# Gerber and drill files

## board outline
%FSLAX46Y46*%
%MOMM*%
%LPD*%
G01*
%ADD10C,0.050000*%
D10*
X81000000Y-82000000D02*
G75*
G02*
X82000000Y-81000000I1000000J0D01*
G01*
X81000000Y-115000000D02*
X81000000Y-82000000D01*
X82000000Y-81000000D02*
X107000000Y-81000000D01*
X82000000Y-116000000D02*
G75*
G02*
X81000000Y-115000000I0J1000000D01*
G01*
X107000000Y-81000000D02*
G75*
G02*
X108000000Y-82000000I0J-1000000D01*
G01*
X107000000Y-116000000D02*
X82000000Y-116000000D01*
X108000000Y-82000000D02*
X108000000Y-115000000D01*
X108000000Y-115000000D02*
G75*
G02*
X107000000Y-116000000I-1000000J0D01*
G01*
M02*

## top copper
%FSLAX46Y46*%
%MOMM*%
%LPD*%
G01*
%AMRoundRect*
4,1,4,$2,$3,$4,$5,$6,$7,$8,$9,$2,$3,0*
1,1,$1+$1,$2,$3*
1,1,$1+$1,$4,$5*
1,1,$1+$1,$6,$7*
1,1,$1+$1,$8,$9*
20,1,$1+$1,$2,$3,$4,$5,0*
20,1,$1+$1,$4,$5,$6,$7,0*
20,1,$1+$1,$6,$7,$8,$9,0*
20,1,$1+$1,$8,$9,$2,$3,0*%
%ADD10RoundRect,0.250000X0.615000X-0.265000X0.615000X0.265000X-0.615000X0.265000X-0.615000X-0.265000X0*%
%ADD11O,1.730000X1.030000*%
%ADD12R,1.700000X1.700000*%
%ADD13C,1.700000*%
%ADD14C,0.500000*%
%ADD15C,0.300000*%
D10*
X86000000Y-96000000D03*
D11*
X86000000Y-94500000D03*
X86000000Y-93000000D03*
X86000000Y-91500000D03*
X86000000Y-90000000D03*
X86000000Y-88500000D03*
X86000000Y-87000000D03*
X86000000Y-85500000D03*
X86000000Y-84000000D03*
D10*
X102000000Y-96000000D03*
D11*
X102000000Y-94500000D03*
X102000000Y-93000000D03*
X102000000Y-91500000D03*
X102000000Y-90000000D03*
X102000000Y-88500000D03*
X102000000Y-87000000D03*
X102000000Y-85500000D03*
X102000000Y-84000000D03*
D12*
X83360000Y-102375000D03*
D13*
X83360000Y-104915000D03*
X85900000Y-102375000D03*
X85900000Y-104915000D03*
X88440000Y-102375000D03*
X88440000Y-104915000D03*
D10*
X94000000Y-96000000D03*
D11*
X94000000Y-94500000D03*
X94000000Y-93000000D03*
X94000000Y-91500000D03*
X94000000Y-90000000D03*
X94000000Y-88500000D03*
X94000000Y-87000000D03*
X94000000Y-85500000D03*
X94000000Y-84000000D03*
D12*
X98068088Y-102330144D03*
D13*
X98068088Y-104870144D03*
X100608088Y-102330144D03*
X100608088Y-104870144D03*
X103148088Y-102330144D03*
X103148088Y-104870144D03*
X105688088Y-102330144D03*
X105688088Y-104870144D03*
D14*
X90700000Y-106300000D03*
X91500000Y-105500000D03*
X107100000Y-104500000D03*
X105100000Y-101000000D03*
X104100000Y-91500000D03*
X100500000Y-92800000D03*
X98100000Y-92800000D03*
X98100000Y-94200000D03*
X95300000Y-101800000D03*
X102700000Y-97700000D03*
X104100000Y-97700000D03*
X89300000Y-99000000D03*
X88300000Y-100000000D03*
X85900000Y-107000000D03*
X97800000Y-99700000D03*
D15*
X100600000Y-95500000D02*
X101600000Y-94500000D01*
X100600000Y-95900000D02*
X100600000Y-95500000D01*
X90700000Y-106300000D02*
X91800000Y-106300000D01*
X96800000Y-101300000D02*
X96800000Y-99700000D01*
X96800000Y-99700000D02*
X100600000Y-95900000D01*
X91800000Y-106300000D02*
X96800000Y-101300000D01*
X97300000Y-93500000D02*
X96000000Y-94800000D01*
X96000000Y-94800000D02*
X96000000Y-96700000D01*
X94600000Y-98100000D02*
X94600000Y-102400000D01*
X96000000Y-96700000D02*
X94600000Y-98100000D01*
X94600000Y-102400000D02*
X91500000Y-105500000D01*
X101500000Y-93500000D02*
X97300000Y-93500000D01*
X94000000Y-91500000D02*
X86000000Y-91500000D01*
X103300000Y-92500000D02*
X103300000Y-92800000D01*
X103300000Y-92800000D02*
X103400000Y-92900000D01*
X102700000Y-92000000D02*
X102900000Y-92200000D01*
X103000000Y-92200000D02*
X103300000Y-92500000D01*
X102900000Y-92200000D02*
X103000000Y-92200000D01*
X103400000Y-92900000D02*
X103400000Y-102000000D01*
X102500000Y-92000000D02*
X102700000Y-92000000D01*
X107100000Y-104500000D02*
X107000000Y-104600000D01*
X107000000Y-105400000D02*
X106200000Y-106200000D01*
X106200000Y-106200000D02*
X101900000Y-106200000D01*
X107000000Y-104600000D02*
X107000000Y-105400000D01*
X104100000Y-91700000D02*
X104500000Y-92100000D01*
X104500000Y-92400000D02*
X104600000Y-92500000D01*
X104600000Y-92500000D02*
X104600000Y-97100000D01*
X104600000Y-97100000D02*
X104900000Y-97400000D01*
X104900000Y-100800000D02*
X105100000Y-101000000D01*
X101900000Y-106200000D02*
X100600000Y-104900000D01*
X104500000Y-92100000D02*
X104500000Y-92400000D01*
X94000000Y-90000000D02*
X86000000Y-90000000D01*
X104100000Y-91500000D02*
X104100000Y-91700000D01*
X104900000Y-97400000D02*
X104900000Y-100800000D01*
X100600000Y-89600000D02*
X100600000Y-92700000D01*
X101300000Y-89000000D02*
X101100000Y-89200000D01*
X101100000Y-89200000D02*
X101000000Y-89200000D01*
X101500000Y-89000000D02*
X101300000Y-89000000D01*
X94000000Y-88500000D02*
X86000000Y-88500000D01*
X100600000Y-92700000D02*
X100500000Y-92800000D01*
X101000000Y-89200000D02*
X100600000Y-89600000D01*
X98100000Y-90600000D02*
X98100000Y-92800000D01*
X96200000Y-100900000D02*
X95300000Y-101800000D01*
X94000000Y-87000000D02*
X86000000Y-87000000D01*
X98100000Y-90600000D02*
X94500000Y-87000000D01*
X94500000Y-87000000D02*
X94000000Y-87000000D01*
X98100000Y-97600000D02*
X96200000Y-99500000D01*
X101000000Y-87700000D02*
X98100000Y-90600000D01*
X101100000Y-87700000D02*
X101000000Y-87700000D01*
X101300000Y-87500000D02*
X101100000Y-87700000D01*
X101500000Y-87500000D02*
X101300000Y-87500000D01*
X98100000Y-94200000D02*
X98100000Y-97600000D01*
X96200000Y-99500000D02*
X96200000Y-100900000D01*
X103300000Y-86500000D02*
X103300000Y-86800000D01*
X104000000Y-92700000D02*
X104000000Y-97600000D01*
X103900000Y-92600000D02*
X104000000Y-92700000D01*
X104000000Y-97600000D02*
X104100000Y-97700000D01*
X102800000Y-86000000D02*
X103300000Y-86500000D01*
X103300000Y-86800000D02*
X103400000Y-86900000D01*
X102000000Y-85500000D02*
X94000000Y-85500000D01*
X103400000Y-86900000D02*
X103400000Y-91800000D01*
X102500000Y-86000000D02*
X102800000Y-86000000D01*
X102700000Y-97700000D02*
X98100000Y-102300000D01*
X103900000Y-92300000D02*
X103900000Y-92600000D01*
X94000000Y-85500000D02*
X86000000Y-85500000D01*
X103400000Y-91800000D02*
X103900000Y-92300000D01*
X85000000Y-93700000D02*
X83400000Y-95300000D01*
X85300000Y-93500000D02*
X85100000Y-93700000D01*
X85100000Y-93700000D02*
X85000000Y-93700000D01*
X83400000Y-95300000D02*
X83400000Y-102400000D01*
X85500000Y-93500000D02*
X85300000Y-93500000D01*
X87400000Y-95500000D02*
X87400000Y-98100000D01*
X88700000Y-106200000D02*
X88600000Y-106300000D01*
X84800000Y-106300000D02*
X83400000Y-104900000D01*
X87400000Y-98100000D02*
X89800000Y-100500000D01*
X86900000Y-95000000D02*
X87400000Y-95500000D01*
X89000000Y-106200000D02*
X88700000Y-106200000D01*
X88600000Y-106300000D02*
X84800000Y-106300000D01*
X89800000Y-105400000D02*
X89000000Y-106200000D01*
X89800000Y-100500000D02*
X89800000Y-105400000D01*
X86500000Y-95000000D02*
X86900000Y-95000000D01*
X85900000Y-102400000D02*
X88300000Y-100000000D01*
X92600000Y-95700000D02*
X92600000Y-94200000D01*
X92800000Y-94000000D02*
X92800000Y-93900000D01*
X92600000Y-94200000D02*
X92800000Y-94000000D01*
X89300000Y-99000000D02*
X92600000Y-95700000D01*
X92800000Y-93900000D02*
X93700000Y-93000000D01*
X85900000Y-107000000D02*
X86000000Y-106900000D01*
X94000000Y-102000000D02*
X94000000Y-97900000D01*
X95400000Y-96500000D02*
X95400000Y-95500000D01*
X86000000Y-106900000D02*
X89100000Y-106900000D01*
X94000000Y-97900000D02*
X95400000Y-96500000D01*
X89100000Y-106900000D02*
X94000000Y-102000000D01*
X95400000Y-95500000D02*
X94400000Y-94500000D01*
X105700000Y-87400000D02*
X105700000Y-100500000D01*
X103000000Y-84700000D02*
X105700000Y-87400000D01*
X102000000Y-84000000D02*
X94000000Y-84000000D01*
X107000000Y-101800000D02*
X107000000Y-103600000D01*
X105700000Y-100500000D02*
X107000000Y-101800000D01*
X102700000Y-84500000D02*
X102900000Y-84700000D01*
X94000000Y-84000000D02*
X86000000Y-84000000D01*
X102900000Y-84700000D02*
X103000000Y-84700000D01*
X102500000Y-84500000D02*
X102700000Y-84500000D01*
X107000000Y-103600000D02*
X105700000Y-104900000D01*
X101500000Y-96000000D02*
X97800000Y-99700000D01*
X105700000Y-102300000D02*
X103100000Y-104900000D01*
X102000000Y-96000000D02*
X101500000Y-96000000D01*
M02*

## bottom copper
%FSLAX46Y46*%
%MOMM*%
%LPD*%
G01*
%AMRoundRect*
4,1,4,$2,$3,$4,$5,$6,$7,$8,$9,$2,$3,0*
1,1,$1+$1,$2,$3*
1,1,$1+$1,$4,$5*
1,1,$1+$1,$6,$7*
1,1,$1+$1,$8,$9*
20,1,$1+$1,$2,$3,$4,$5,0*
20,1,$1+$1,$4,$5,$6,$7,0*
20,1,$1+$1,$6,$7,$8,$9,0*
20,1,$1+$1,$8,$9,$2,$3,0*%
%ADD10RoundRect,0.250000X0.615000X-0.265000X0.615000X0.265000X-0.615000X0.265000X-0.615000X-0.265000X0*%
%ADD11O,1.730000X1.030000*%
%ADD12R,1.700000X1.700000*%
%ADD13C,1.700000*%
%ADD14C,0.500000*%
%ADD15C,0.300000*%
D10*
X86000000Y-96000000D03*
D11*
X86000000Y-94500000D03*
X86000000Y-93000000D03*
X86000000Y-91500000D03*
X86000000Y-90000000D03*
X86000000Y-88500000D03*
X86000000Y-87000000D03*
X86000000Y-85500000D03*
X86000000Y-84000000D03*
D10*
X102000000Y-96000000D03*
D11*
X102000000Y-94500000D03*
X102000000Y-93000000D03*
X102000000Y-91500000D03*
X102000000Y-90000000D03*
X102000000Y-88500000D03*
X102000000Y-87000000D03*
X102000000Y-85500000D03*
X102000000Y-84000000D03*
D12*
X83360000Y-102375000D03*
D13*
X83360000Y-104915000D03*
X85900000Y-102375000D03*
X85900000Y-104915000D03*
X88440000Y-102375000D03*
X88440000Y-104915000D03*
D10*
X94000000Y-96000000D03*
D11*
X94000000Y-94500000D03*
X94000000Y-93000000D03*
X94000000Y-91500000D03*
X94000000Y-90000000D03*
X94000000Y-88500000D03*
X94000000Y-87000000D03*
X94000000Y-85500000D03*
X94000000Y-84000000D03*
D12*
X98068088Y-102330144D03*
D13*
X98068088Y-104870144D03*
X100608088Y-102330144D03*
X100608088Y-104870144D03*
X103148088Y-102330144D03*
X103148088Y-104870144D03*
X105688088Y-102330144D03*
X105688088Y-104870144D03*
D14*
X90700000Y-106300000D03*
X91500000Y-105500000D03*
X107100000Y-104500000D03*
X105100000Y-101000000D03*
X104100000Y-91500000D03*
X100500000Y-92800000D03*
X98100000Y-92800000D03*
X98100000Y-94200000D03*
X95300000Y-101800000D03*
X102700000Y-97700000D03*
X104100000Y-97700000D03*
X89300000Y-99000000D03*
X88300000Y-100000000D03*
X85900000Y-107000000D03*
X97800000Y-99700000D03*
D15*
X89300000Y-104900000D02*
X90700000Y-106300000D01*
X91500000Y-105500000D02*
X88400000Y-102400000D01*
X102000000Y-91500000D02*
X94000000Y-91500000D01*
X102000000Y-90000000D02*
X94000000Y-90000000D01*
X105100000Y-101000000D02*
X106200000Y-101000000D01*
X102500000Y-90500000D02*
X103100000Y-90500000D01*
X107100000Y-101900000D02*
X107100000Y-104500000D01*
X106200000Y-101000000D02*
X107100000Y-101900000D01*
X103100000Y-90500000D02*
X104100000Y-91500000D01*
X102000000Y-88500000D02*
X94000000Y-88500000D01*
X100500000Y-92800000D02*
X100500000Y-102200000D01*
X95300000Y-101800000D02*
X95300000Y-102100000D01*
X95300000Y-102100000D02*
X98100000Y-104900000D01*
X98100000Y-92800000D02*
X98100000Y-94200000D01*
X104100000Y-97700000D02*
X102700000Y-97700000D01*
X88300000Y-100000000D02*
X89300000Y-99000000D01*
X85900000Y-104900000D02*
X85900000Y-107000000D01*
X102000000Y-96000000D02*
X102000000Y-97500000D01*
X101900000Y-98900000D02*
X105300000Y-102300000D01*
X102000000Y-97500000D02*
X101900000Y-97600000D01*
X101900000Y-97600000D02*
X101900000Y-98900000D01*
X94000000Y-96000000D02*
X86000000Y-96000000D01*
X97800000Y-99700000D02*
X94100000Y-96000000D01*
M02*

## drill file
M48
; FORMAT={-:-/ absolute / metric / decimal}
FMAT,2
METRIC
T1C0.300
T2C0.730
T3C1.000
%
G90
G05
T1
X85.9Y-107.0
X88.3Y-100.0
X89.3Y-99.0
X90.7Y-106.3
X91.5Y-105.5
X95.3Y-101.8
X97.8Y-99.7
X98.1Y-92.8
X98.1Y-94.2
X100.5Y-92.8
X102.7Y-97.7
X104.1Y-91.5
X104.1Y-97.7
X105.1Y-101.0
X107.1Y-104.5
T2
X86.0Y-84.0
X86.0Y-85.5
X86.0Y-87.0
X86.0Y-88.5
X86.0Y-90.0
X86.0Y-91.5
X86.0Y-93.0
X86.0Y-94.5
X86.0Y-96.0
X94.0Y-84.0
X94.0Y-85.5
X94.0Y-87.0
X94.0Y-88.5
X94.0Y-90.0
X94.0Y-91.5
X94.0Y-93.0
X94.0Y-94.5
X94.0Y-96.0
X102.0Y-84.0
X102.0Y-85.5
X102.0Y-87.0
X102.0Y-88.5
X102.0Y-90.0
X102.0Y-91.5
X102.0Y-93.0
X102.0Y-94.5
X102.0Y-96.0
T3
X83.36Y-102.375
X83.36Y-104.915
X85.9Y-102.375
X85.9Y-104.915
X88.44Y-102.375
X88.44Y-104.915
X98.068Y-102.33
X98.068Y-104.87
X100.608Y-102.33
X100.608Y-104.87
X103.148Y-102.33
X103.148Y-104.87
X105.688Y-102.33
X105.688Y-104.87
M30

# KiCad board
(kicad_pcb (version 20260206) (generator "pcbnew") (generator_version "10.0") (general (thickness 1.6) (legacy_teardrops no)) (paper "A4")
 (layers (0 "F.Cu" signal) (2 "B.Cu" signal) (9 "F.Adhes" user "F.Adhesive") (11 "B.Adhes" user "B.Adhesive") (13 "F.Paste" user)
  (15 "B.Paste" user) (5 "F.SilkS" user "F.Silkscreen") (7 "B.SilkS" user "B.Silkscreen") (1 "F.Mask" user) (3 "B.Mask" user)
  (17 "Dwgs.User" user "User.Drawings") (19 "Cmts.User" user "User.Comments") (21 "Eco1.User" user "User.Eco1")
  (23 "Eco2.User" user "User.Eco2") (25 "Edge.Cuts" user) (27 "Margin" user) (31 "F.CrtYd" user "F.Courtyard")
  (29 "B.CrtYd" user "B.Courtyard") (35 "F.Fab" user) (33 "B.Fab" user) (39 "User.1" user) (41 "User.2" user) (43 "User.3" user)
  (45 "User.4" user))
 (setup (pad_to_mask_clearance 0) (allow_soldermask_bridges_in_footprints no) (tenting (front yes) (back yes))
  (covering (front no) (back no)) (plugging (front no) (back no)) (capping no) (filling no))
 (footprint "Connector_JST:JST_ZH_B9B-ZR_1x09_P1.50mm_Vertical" (layer "F.Cu") (at 86 96 90)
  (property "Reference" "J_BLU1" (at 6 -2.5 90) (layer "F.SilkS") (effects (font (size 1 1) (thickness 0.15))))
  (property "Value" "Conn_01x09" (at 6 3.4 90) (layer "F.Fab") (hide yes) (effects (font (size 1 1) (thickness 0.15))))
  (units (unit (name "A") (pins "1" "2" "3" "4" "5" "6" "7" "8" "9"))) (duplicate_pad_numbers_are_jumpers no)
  (pad "1" thru_hole roundrect (at 0 0 90) (size 1.03 1.73) (drill 0.73) (layers "*.Cu" "*.Mask") (remove_unused_layers no)
   (roundrect_rratio 0.242718) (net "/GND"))
  (pad "2" thru_hole oval (at 1.5 0 90) (size 1.03 1.73) (drill 0.73) (layers "*.Cu" "*.Mask") (remove_unused_layers no) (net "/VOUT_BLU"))
  (pad "3" thru_hole oval (at 3 0 90) (size 1.03 1.73) (drill 0.73) (layers "*.Cu" "*.Mask") (remove_unused_layers no) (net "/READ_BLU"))
  (pad "4" thru_hole oval (at 4.5 0 90) (size 1.03 1.73) (drill 0.73) (layers "*.Cu" "*.Mask") (remove_unused_layers no) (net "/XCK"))
  (pad "5" thru_hole oval (at 6 0 90) (size 1.03 1.73) (drill 0.73) (layers "*.Cu" "*.Mask") (remove_unused_layers no) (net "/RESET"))
  (pad "6" thru_hole oval (at 7.5 0 90) (size 1.03 1.73) (drill 0.73) (layers "*.Cu" "*.Mask") (remove_unused_layers no) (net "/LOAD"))
  (pad "7" thru_hole oval (at 9 0 90) (size 1.03 1.73) (drill 0.73) (layers "*.Cu" "*.Mask") (remove_unused_layers no) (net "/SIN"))
  (pad "8" thru_hole oval (at 10.5 0 90) (size 1.03 1.73) (drill 0.73) (layers "*.Cu" "*.Mask") (remove_unused_layers no) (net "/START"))
  (pad "9" thru_hole oval (at 12 0 90) (size 1.03 1.73) (drill 0.73) (layers "*.Cu" "*.Mask") (remove_unused_layers no) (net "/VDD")))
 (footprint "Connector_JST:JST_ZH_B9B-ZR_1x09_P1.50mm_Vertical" (layer "F.Cu") (at 102 96 90)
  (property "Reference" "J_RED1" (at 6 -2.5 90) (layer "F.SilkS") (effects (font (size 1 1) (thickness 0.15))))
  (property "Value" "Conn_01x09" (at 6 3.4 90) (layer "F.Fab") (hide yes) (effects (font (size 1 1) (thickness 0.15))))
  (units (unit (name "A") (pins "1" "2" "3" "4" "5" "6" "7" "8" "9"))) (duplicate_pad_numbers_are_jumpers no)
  (pad "1" thru_hole roundrect (at 0 0 90) (size 1.03 1.73) (drill 0.73) (layers "*.Cu" "*.Mask") (remove_unused_layers no)
   (roundrect_rratio 0.242718) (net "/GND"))
  (pad "2" thru_hole oval (at 1.5 0 90) (size 1.03 1.73) (drill 0.73) (layers "*.Cu" "*.Mask") (remove_unused_layers no) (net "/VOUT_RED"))
  (pad "3" thru_hole oval (at 3 0 90) (size 1.03 1.73) (drill 0.73) (layers "*.Cu" "*.Mask") (remove_unused_layers no) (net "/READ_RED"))
  (pad "4" thru_hole oval (at 4.5 0 90) (size 1.03 1.73) (drill 0.73) (layers "*.Cu" "*.Mask") (remove_unused_layers no) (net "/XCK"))
  (pad "5" thru_hole oval (at 6 0 90) (size 1.03 1.73) (drill 0.73) (layers "*.Cu" "*.Mask") (remove_unused_layers no) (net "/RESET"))
  (pad "6" thru_hole oval (at 7.5 0 90) (size 1.03 1.73) (drill 0.73) (layers "*.Cu" "*.Mask") (remove_unused_layers no) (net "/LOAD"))
  (pad "7" thru_hole oval (at 9 0 90) (size 1.03 1.73) (drill 0.73) (layers "*.Cu" "*.Mask") (remove_unused_layers no) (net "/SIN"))
  (pad "8" thru_hole oval (at 10.5 0 90) (size 1.03 1.73) (drill 0.73) (layers "*.Cu" "*.Mask") (remove_unused_layers no) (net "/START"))
  (pad "9" thru_hole oval (at 12 0 90) (size 1.03 1.73) (drill 0.73) (layers "*.Cu" "*.Mask") (remove_unused_layers no) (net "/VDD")))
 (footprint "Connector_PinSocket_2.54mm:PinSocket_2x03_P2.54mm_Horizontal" (layer "F.Cu") (at 83.36 102.375 90)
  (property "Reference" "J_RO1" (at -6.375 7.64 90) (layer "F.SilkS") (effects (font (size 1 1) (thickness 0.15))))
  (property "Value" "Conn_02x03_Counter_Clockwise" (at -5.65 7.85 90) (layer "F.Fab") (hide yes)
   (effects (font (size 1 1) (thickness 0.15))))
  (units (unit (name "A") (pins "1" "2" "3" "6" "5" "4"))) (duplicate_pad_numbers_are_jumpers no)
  (pad "1" thru_hole rect (at 0 0 90) (size 1.7 1.7) (drill 1) (layers "*.Cu" "*.Mask") (remove_unused_layers no) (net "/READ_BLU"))
  (pad "2" thru_hole circle (at -2.54 0 90) (size 1.7 1.7) (drill 1) (layers "*.Cu" "*.Mask") (remove_unused_layers no) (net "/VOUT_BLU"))
  (pad "3" thru_hole circle (at 0 2.54 90) (size 1.7 1.7) (drill 1) (layers "*.Cu" "*.Mask") (remove_unused_layers no) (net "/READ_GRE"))
  (pad "4" thru_hole circle (at -2.54 2.54 90) (size 1.7 1.7) (drill 1) (layers "*.Cu" "*.Mask") (remove_unused_layers no) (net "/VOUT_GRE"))
  (pad "5" thru_hole circle (at 0 5.08 90) (size 1.7 1.7) (drill 1) (layers "*.Cu" "*.Mask") (remove_unused_layers no) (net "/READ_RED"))
  (pad "6" thru_hole circle (at -2.54 5.08 90) (size 1.7 1.7) (drill 1) (layers "*.Cu" "*.Mask") (remove_unused_layers no) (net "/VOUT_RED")))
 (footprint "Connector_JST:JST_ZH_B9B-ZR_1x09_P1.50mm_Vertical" (layer "F.Cu") (at 94 96 90)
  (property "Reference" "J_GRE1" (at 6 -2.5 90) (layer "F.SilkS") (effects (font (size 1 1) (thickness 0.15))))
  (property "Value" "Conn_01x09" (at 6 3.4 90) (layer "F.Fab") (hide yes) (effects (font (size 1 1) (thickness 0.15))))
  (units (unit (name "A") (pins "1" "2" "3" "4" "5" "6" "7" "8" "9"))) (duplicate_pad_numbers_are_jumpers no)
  (pad "1" thru_hole roundrect (at 0 0 90) (size 1.03 1.73) (drill 0.73) (layers "*.Cu" "*.Mask") (remove_unused_layers no)
   (roundrect_rratio 0.242718) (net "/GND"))
  (pad "2" thru_hole oval (at 1.5 0 90) (size 1.03 1.73) (drill 0.73) (layers "*.Cu" "*.Mask") (remove_unused_layers no) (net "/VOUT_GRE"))
  (pad "3" thru_hole oval (at 3 0 90) (size 1.03 1.73) (drill 0.73) (layers "*.Cu" "*.Mask") (remove_unused_layers no) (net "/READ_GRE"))
  (pad "4" thru_hole oval (at 4.5 0 90) (size 1.03 1.73) (drill 0.73) (layers "*.Cu" "*.Mask") (remove_unused_layers no) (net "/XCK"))
  (pad "5" thru_hole oval (at 6 0 90) (size 1.03 1.73) (drill 0.73) (layers "*.Cu" "*.Mask") (remove_unused_layers no) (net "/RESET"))
  (pad "6" thru_hole oval (at 7.5 0 90) (size 1.03 1.73) (drill 0.73) (layers "*.Cu" "*.Mask") (remove_unused_layers no) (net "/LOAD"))
  (pad "7" thru_hole oval (at 9 0 90) (size 1.03 1.73) (drill 0.73) (layers "*.Cu" "*.Mask") (remove_unused_layers no) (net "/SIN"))
  (pad "8" thru_hole oval (at 10.5 0 90) (size 1.03 1.73) (drill 0.73) (layers "*.Cu" "*.Mask") (remove_unused_layers no) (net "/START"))
  (pad "9" thru_hole oval (at 12 0 90) (size 1.03 1.73) (drill 0.73) (layers "*.Cu" "*.Mask") (remove_unused_layers no) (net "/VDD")))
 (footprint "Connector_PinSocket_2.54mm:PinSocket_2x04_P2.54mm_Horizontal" (layer "F.Cu") (at 98.068088 102.330144 90)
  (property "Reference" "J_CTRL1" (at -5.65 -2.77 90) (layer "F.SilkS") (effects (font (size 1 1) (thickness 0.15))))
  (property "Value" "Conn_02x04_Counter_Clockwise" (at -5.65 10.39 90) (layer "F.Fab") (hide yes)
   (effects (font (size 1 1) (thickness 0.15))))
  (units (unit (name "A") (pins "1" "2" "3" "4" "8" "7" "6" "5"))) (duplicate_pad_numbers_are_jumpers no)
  (pad "1" thru_hole rect (at 0 0 90) (size 1.7 1.7) (drill 1) (layers "*.Cu" "*.Mask") (remove_unused_layers no) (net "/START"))
  (pad "2" thru_hole circle (at -2.54 0 90) (size 1.7 1.7) (drill 1) (layers "*.Cu" "*.Mask") (remove_unused_layers no) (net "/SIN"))
  (pad "3" thru_hole circle (at 0 2.54 90) (size 1.7 1.7) (drill 1) (layers "*.Cu" "*.Mask") (remove_unused_layers no) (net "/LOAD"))
  (pad "4" thru_hole circle (at -2.54 2.54 90) (size 1.7 1.7) (drill 1) (layers "*.Cu" "*.Mask") (remove_unused_layers no) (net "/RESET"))
  (pad "5" thru_hole circle (at 0 5.08 90) (size 1.7 1.7) (drill 1) (layers "*.Cu" "*.Mask") (remove_unused_layers no) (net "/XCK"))
  (pad "6" thru_hole circle (at -2.54 5.08 90) (size 1.7 1.7) (drill 1) (layers "*.Cu" "*.Mask") (remove_unused_layers no) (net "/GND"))
  (pad "7" thru_hole circle (at 0 7.62 90) (size 1.7 1.7) (drill 1) (layers "*.Cu" "*.Mask") (remove_unused_layers no) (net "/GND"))
  (pad "8" thru_hole circle (at -2.54 7.62 90) (size 1.7 1.7) (drill 1) (layers "*.Cu" "*.Mask") (remove_unused_layers no) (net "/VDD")))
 (gr_arc (start 81 82) (mid 81.292893 81.292893) (end 82 81) (stroke (width 0.05) (type default)) (layer "Edge.Cuts"))
 (gr_line (start 81 115) (end 81 82) (stroke (width 0.05) (type default)) (layer "Edge.Cuts"))
 (gr_line (start 82 81) (end 107 81) (stroke (width 0.05) (type default)) (layer "Edge.Cuts"))
 (gr_arc (start 82 116) (mid 81.292893 115.707107) (end 81 115) (stroke (width 0.05) (type default)) (layer "Edge.Cuts"))
 (gr_arc (start 107 81) (mid 107.707107 81.292893) (end 108 82) (stroke (width 0.05) (type default)) (layer "Edge.Cuts"))
 (gr_line (start 107 116) (end 82 116) (stroke (width 0.05) (type default)) (layer "Edge.Cuts"))
 (gr_line (start 108 82) (end 108 115) (stroke (width 0.05) (type default)) (layer "Edge.Cuts"))
 (gr_arc (start 108 115) (mid 107.707107 115.707107) (end 107 116) (stroke (width 0.05) (type default)) (layer "Edge.Cuts"))
 (segment (start 100.6 95.5) (end 101.6 94.5) (width 0.3) (layer "F.Cu") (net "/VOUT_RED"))
 (segment (start 100.6 95.9) (end 100.6 95.5) (width 0.3) (layer "F.Cu") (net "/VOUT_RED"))
 (segment (start 90.7 106.3) (end 91.8 106.3) (width 0.3) (layer "F.Cu") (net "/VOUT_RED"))
 (segment (start 96.8 101.3) (end 96.8 99.7) (width 0.3) (layer "F.Cu") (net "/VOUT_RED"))
 (segment (start 96.8 99.7) (end 100.6 95.9) (width 0.3) (layer "F.Cu") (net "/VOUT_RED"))
 (segment (start 91.8 106.3) (end 96.8 101.3) (width 0.3) (layer "F.Cu") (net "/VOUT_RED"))
 (via (at 90.7 106.3) (size 0.5) (drill 0.3) (layers "F.Cu" "B.Cu") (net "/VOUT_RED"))
 (segment (start 89.3 104.9) (end 90.7 106.3) (width 0.3) (layer "B.Cu") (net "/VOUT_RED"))
 (segment (start 97.3 93.5) (end 96 94.8) (width 0.3) (layer "F.Cu") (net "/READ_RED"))
 (segment (start 96 94.8) (end 96 96.7) (width 0.3) (layer "F.Cu") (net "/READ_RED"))
 (segment (start 94.6 98.1) (end 94.6 102.4) (width 0.3) (layer "F.Cu") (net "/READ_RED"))
 (segment (start 96 96.7) (end 94.6 98.1) (width 0.3) (layer "F.Cu") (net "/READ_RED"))
 (segment (start 94.6 102.4) (end 91.5 105.5) (width 0.3) (layer "F.Cu") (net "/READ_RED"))
 (segment (start 101.5 93.5) (end 97.3 93.5) (width 0.3) (layer "F.Cu") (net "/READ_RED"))
 (via (at 91.5 105.5) (size 0.5) (drill 0.3) (layers "F.Cu" "B.Cu") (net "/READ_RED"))
 (segment (start 91.5 105.5) (end 88.4 102.4) (width 0.3) (layer "B.Cu") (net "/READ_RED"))
 (segment (start 94 91.5) (end 86 91.5) (width 0.3) (layer "F.Cu") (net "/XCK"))
 (segment (start 103.3 92.5) (end 103.3 92.8) (width 0.3) (layer "F.Cu") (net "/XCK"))
 (segment (start 103.3 92.8) (end 103.4 92.9) (width 0.3) (layer "F.Cu") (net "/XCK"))
 (segment (start 102.7 92) (end 102.9 92.2) (width 0.3) (layer "F.Cu") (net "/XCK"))
 (segment (start 103 92.2) (end 103.3 92.5) (width 0.3) (layer "F.Cu") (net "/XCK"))
 (segment (start 102.9 92.2) (end 103 92.2) (width 0.3) (layer "F.Cu") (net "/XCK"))
 (segment (start 103.4 92.9) (end 103.4 102) (width 0.3) (layer "F.Cu") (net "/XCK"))
 (segment (start 102.5 92) (end 102.7 92) (width 0.3) (layer "F.Cu") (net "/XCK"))
 (segment (start 102 91.5) (end 94 91.5) (width 0.3) (layer "B.Cu") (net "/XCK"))
 (segment (start 107.1 104.5) (end 107 104.6) (width 0.3) (layer "F.Cu") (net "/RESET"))
 (segment (start 107 105.4) (end 106.2 106.2) (width 0.3) (layer "F.Cu") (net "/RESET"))
 (segment (start 106.2 106.2) (end 101.9 106.2) (width 0.3) (layer "F.Cu") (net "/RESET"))
 (segment (start 107 104.6) (end 107 105.4) (width 0.3) (layer "F.Cu") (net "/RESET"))
 (segment (start 104.1 91.7) (end 104.5 92.1) (width 0.3) (layer "F.Cu") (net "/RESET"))
 (segment (start 104.5 92.4) (end 104.6 92.5) (width 0.3) (layer "F.Cu") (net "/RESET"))
 (segment (start 104.6 92.5) (end 104.6 97.1) (width 0.3) (layer "F.Cu") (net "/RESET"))
 (segment (start 104.6 97.1) (end 104.9 97.4) (width 0.3) (layer "F.Cu") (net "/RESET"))
 (segment (start 104.9 100.8) (end 105.1 101) (width 0.3) (layer "F.Cu") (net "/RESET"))
 (segment (start 101.9 106.2) (end 100.6 104.9) (width 0.3) (layer "F.Cu") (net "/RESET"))
 (segment (start 104.5 92.1) (end 104.5 92.4) (width 0.3) (layer "F.Cu") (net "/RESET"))
 (segment (start 94 90) (end 86 90) (width 0.3) (layer "F.Cu") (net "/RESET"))
 (segment (start 104.1 91.5) (end 104.1 91.7) (width 0.3) (layer "F.Cu") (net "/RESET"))
 (segment (start 104.9 97.4) (end 104.9 100.8) (width 0.3) (layer "F.Cu") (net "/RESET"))
 (via (at 107.1 104.5) (size 0.5) (drill 0.3) (layers "F.Cu" "B.Cu") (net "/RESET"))
 (via (at 105.1 101) (size 0.5) (drill 0.3) (layers "F.Cu" "B.Cu") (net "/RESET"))
 (via (at 104.1 91.5) (size 0.5) (drill 0.3) (layers "F.Cu" "B.Cu") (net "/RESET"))
 (segment (start 102 90) (end 94 90) (width 0.3) (layer "B.Cu") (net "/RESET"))
 (segment (start 105.1 101) (end 106.2 101) (width 0.3) (layer "B.Cu") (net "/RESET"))
 (segment (start 102.5 90.5) (end 103.1 90.5) (width 0.3) (layer "B.Cu") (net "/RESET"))
 (segment (start 107.1 101.9) (end 107.1 104.5) (width 0.3) (layer "B.Cu") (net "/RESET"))
 (segment (start 106.2 101) (end 107.1 101.9) (width 0.3) (layer "B.Cu") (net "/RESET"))
 (segment (start 103.1 90.5) (end 104.1 91.5) (width 0.3) (layer "B.Cu") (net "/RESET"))
 (segment (start 100.6 89.6) (end 100.6 92.7) (width 0.3) (layer "F.Cu") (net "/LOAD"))
 (segment (start 101.3 89) (end 101.1 89.2) (width 0.3) (layer "F.Cu") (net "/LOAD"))
 (segment (start 101.1 89.2) (end 101 89.2) (width 0.3) (layer "F.Cu") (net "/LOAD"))
 (segment (start 101.5 89) (end 101.3 89) (width 0.3) (layer "F.Cu") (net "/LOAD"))
 (segment (start 94 88.5) (end 86 88.5) (width 0.3) (layer "F.Cu") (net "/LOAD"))
 (segment (start 100.6 92.7) (end 100.5 92.8) (width 0.3) (layer "F.Cu") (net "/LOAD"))
 (segment (start 101 89.2) (end 100.6 89.6) (width 0.3) (layer "F.Cu") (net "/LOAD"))
 (via (at 100.5 92.8) (size 0.5) (drill 0.3) (layers "F.Cu" "B.Cu") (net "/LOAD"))
 (segment (start 102 88.5) (end 94 88.5) (width 0.3) (layer "B.Cu") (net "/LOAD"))
 (segment (start 100.5 92.8) (end 100.5 102.2) (width 0.3) (layer "B.Cu") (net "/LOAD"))
 (segment (start 98.1 90.6) (end 98.1 92.8) (width 0.3) (layer "F.Cu") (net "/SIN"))
 (segment (start 96.2 100.9) (end 95.3 101.8) (width 0.3) (layer "F.Cu") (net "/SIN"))
 (segment (start 94 87) (end 86 87) (width 0.3) (layer "F.Cu") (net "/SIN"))
 (segment (start 98.1 90.6) (end 94.5 87) (width 0.3) (layer "F.Cu") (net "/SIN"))
 (segment (start 94.5 87) (end 94 87) (width 0.3) (layer "F.Cu") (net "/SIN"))
 (segment (start 98.1 97.6) (end 96.2 99.5) (width 0.3) (layer "F.Cu") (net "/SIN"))
 (segment (start 101 87.7) (end 98.1 90.6) (width 0.3) (layer "F.Cu") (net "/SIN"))
 (segment (start 101.1 87.7) (end 101 87.7) (width 0.3) (layer "F.Cu") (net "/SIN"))
 (segment (start 101.3 87.5) (end 101.1 87.7) (width 0.3) (layer "F.Cu") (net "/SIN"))
 (segment (start 101.5 87.5) (end 101.3 87.5) (width 0.3) (layer "F.Cu") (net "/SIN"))
 (segment (start 98.1 94.2) (end 98.1 97.6) (width 0.3) (layer "F.Cu") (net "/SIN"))
 (segment (start 96.2 99.5) (end 96.2 100.9) (width 0.3) (layer "F.Cu") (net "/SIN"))
 (via (at 98.1 92.8) (size 0.5) (drill 0.3) (layers "F.Cu" "B.Cu") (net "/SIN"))
 (via (at 98.1 94.2) (size 0.5) (drill 0.3) (layers "F.Cu" "B.Cu") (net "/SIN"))
 (via (at 95.3 101.8) (size 0.5) (drill 0.3) (layers "F.Cu" "B.Cu") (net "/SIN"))
 (segment (start 95.3 101.8) (end 95.3 102.1) (width 0.3) (layer "B.Cu") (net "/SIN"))
 (segment (start 95.3 102.1) (end 98.1 104.9) (width 0.3) (layer "B.Cu") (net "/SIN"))
 (segment (start 98.1 92.8) (end 98.1 94.2) (width 0.3) (layer "B.Cu") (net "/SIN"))
 (segment (start 103.3 86.5) (end 103.3 86.8) (width 0.3) (layer "F.Cu") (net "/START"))
 (segment (start 104 92.7) (end 104 97.6) (width 0.3) (layer "F.Cu") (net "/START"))
 (segment (start 103.9 92.6) (end 104 92.7) (width 0.3) (layer "F.Cu") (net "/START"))
 (segment (start 104 97.6) (end 104.1 97.7) (width 0.3) (layer "F.Cu") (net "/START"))
 (segment (start 102.8 86) (end 103.3 86.5) (width 0.3) (layer "F.Cu") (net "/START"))
 (segment (start 103.3 86.8) (end 103.4 86.9) (width 0.3) (layer "F.Cu") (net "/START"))
 (segment (start 102 85.5) (end 94 85.5) (width 0.3) (layer "F.Cu") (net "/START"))
 (segment (start 103.4 86.9) (end 103.4 91.8) (width 0.3) (layer "F.Cu") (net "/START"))
 (segment (start 102.5 86) (end 102.8 86) (width 0.3) (layer "F.Cu") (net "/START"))
 (segment (start 102.7 97.7) (end 98.1 102.3) (width 0.3) (layer "F.Cu") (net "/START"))
 (segment (start 103.9 92.3) (end 103.9 92.6) (width 0.3) (layer "F.Cu") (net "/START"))
 (segment (start 94 85.5) (end 86 85.5) (width 0.3) (layer "F.Cu") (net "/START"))
 (segment (start 103.4 91.8) (end 103.9 92.3) (width 0.3) (layer "F.Cu") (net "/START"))
 (via (at 102.7 97.7) (size 0.5) (drill 0.3) (layers "F.Cu" "B.Cu") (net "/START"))
 (via (at 104.1 97.7) (size 0.5) (drill 0.3) (layers "F.Cu" "B.Cu") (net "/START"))
 (segment (start 104.1 97.7) (end 102.7 97.7) (width 0.3) (layer "B.Cu") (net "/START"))
 (segment (start 85 93.7) (end 83.4 95.3) (width 0.3) (layer "F.Cu") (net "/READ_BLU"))
 (segment (start 85.3 93.5) (end 85.1 93.7) (width 0.3) (layer "F.Cu") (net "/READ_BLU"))
 (segment (start 85.1 93.7) (end 85 93.7) (width 0.3) (layer "F.Cu") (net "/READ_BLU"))
 (segment (start 83.4 95.3) (end 83.4 102.4) (width 0.3) (layer "F.Cu") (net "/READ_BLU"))
 (segment (start 85.5 93.5) (end 85.3 93.5) (width 0.3) (layer "F.Cu") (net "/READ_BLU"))
 (segment (start 87.4 95.5) (end 87.4 98.1) (width 0.3) (layer "F.Cu") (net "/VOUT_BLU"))
 (segment (start 88.7 106.2) (end 88.6 106.3) (width 0.3) (layer "F.Cu") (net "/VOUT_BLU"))
 (segment (start 84.8 106.3) (end 83.4 104.9) (width 0.3) (layer "F.Cu") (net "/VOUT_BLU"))
 (segment (start 87.4 98.1) (end 89.8 100.5) (width 0.3) (layer "F.Cu") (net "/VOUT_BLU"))
 (segment (start 86.9 95) (end 87.4 95.5) (width 0.3) (layer "F.Cu") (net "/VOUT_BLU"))
 (segment (start 89 106.2) (end 88.7 106.2) (width 0.3) (layer "F.Cu") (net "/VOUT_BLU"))
 (segment (start 88.6 106.3) (end 84.8 106.3) (width 0.3) (layer "F.Cu") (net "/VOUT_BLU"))
 (segment (start 89.8 105.4) (end 89 106.2) (width 0.3) (layer "F.Cu") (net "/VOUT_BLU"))
 (segment (start 89.8 100.5) (end 89.8 105.4) (width 0.3) (layer "F.Cu") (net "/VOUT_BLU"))
 (segment (start 86.5 95) (end 86.9 95) (width 0.3) (layer "F.Cu") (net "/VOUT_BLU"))
 (segment (start 85.9 102.4) (end 88.3 100) (width 0.3) (layer "F.Cu") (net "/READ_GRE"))
 (segment (start 92.6 95.7) (end 92.6 94.2) (width 0.3) (layer "F.Cu") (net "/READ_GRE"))
 (segment (start 92.8 94) (end 92.8 93.9) (width 0.3) (layer "F.Cu") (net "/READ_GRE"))
 (segment (start 92.6 94.2) (end 92.8 94) (width 0.3) (layer "F.Cu") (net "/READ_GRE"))
 (segment (start 89.3 99) (end 92.6 95.7) (width 0.3) (layer "F.Cu") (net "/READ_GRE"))
 (segment (start 92.8 93.9) (end 93.7 93) (width 0.3) (layer "F.Cu") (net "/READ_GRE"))
 (via (at 89.3 99) (size 0.5) (drill 0.3) (layers "F.Cu" "B.Cu") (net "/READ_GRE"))
 (via (at 88.3 100) (size 0.5) (drill 0.3) (layers "F.Cu" "B.Cu") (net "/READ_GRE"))
 (segment (start 88.3 100) (end 89.3 99) (width 0.3) (layer "B.Cu") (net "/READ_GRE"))
 (segment (start 85.9 107) (end 86 106.9) (width 0.3) (layer "F.Cu") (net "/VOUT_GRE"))
 (segment (start 94 102) (end 94 97.9) (width 0.3) (layer "F.Cu") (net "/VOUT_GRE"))
 (segment (start 95.4 96.5) (end 95.4 95.5) (width 0.3) (layer "F.Cu") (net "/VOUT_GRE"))
 (segment (start 86 106.9) (end 89.1 106.9) (width 0.3) (layer "F.Cu") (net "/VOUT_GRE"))
 (segment (start 94 97.9) (end 95.4 96.5) (width 0.3) (layer "F.Cu") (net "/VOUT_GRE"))
 (segment (start 89.1 106.9) (end 94 102) (width 0.3) (layer "F.Cu") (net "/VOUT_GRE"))
 (segment (start 95.4 95.5) (end 94.4 94.5) (width 0.3) (layer "F.Cu") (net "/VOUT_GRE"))
 (via (at 85.9 107) (size 0.5) (drill 0.3) (layers "F.Cu" "B.Cu") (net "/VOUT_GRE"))
 (segment (start 85.9 104.9) (end 85.9 107) (width 0.3) (layer "B.Cu") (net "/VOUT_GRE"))
 (segment (start 105.7 87.4) (end 105.7 100.5) (width 0.3) (layer "F.Cu") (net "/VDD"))
 (segment (start 103 84.7) (end 105.7 87.4) (width 0.3) (layer "F.Cu") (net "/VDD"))
 (segment (start 102 84) (end 94 84) (width 0.3) (layer "F.Cu") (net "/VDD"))
 (segment (start 107 101.8) (end 107 103.6) (width 0.3) (layer "F.Cu") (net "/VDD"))
 (segment (start 105.7 100.5) (end 107 101.8) (width 0.3) (layer "F.Cu") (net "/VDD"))
 (segment (start 102.7 84.5) (end 102.9 84.7) (width 0.3) (layer "F.Cu") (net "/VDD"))
 (segment (start 94 84) (end 86 84) (width 0.3) (layer "F.Cu") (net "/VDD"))
 (segment (start 102.9 84.7) (end 103 84.7) (width 0.3) (layer "F.Cu") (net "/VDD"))
 (segment (start 102.5 84.5) (end 102.7 84.5) (width 0.3) (layer "F.Cu") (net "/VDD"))
 (segment (start 107 103.6) (end 105.7 104.9) (width 0.3) (layer "F.Cu") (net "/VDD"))
 (segment (start 101.5 96) (end 97.8 99.7) (width 0.3) (layer "F.Cu") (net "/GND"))
 (segment (start 105.7 102.3) (end 103.1 104.9) (width 0.3) (layer "F.Cu") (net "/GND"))
 (segment (start 102 96) (end 101.5 96) (width 0.3) (layer "F.Cu") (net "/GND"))
 (via (at 97.8 99.7) (size 0.5) (drill 0.3) (layers "F.Cu" "B.Cu") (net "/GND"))
 (segment (start 102 96) (end 102 97.5) (width 0.3) (layer "B.Cu") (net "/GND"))
 (segment (start 101.9 98.9) (end 105.3 102.3) (width 0.3) (layer "B.Cu") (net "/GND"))
 (segment (start 102 97.5) (end 101.9 97.6) (width 0.3) (layer "B.Cu") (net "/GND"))
 (segment (start 101.9 97.6) (end 101.9 98.9) (width 0.3) (layer "B.Cu") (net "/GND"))
 (segment (start 94 96) (end 86 96) (width 0.3) (layer "B.Cu") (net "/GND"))
 (segment (start 97.8 99.7) (end 94.1 96) (width 0.3) (layer "B.Cu") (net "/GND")))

